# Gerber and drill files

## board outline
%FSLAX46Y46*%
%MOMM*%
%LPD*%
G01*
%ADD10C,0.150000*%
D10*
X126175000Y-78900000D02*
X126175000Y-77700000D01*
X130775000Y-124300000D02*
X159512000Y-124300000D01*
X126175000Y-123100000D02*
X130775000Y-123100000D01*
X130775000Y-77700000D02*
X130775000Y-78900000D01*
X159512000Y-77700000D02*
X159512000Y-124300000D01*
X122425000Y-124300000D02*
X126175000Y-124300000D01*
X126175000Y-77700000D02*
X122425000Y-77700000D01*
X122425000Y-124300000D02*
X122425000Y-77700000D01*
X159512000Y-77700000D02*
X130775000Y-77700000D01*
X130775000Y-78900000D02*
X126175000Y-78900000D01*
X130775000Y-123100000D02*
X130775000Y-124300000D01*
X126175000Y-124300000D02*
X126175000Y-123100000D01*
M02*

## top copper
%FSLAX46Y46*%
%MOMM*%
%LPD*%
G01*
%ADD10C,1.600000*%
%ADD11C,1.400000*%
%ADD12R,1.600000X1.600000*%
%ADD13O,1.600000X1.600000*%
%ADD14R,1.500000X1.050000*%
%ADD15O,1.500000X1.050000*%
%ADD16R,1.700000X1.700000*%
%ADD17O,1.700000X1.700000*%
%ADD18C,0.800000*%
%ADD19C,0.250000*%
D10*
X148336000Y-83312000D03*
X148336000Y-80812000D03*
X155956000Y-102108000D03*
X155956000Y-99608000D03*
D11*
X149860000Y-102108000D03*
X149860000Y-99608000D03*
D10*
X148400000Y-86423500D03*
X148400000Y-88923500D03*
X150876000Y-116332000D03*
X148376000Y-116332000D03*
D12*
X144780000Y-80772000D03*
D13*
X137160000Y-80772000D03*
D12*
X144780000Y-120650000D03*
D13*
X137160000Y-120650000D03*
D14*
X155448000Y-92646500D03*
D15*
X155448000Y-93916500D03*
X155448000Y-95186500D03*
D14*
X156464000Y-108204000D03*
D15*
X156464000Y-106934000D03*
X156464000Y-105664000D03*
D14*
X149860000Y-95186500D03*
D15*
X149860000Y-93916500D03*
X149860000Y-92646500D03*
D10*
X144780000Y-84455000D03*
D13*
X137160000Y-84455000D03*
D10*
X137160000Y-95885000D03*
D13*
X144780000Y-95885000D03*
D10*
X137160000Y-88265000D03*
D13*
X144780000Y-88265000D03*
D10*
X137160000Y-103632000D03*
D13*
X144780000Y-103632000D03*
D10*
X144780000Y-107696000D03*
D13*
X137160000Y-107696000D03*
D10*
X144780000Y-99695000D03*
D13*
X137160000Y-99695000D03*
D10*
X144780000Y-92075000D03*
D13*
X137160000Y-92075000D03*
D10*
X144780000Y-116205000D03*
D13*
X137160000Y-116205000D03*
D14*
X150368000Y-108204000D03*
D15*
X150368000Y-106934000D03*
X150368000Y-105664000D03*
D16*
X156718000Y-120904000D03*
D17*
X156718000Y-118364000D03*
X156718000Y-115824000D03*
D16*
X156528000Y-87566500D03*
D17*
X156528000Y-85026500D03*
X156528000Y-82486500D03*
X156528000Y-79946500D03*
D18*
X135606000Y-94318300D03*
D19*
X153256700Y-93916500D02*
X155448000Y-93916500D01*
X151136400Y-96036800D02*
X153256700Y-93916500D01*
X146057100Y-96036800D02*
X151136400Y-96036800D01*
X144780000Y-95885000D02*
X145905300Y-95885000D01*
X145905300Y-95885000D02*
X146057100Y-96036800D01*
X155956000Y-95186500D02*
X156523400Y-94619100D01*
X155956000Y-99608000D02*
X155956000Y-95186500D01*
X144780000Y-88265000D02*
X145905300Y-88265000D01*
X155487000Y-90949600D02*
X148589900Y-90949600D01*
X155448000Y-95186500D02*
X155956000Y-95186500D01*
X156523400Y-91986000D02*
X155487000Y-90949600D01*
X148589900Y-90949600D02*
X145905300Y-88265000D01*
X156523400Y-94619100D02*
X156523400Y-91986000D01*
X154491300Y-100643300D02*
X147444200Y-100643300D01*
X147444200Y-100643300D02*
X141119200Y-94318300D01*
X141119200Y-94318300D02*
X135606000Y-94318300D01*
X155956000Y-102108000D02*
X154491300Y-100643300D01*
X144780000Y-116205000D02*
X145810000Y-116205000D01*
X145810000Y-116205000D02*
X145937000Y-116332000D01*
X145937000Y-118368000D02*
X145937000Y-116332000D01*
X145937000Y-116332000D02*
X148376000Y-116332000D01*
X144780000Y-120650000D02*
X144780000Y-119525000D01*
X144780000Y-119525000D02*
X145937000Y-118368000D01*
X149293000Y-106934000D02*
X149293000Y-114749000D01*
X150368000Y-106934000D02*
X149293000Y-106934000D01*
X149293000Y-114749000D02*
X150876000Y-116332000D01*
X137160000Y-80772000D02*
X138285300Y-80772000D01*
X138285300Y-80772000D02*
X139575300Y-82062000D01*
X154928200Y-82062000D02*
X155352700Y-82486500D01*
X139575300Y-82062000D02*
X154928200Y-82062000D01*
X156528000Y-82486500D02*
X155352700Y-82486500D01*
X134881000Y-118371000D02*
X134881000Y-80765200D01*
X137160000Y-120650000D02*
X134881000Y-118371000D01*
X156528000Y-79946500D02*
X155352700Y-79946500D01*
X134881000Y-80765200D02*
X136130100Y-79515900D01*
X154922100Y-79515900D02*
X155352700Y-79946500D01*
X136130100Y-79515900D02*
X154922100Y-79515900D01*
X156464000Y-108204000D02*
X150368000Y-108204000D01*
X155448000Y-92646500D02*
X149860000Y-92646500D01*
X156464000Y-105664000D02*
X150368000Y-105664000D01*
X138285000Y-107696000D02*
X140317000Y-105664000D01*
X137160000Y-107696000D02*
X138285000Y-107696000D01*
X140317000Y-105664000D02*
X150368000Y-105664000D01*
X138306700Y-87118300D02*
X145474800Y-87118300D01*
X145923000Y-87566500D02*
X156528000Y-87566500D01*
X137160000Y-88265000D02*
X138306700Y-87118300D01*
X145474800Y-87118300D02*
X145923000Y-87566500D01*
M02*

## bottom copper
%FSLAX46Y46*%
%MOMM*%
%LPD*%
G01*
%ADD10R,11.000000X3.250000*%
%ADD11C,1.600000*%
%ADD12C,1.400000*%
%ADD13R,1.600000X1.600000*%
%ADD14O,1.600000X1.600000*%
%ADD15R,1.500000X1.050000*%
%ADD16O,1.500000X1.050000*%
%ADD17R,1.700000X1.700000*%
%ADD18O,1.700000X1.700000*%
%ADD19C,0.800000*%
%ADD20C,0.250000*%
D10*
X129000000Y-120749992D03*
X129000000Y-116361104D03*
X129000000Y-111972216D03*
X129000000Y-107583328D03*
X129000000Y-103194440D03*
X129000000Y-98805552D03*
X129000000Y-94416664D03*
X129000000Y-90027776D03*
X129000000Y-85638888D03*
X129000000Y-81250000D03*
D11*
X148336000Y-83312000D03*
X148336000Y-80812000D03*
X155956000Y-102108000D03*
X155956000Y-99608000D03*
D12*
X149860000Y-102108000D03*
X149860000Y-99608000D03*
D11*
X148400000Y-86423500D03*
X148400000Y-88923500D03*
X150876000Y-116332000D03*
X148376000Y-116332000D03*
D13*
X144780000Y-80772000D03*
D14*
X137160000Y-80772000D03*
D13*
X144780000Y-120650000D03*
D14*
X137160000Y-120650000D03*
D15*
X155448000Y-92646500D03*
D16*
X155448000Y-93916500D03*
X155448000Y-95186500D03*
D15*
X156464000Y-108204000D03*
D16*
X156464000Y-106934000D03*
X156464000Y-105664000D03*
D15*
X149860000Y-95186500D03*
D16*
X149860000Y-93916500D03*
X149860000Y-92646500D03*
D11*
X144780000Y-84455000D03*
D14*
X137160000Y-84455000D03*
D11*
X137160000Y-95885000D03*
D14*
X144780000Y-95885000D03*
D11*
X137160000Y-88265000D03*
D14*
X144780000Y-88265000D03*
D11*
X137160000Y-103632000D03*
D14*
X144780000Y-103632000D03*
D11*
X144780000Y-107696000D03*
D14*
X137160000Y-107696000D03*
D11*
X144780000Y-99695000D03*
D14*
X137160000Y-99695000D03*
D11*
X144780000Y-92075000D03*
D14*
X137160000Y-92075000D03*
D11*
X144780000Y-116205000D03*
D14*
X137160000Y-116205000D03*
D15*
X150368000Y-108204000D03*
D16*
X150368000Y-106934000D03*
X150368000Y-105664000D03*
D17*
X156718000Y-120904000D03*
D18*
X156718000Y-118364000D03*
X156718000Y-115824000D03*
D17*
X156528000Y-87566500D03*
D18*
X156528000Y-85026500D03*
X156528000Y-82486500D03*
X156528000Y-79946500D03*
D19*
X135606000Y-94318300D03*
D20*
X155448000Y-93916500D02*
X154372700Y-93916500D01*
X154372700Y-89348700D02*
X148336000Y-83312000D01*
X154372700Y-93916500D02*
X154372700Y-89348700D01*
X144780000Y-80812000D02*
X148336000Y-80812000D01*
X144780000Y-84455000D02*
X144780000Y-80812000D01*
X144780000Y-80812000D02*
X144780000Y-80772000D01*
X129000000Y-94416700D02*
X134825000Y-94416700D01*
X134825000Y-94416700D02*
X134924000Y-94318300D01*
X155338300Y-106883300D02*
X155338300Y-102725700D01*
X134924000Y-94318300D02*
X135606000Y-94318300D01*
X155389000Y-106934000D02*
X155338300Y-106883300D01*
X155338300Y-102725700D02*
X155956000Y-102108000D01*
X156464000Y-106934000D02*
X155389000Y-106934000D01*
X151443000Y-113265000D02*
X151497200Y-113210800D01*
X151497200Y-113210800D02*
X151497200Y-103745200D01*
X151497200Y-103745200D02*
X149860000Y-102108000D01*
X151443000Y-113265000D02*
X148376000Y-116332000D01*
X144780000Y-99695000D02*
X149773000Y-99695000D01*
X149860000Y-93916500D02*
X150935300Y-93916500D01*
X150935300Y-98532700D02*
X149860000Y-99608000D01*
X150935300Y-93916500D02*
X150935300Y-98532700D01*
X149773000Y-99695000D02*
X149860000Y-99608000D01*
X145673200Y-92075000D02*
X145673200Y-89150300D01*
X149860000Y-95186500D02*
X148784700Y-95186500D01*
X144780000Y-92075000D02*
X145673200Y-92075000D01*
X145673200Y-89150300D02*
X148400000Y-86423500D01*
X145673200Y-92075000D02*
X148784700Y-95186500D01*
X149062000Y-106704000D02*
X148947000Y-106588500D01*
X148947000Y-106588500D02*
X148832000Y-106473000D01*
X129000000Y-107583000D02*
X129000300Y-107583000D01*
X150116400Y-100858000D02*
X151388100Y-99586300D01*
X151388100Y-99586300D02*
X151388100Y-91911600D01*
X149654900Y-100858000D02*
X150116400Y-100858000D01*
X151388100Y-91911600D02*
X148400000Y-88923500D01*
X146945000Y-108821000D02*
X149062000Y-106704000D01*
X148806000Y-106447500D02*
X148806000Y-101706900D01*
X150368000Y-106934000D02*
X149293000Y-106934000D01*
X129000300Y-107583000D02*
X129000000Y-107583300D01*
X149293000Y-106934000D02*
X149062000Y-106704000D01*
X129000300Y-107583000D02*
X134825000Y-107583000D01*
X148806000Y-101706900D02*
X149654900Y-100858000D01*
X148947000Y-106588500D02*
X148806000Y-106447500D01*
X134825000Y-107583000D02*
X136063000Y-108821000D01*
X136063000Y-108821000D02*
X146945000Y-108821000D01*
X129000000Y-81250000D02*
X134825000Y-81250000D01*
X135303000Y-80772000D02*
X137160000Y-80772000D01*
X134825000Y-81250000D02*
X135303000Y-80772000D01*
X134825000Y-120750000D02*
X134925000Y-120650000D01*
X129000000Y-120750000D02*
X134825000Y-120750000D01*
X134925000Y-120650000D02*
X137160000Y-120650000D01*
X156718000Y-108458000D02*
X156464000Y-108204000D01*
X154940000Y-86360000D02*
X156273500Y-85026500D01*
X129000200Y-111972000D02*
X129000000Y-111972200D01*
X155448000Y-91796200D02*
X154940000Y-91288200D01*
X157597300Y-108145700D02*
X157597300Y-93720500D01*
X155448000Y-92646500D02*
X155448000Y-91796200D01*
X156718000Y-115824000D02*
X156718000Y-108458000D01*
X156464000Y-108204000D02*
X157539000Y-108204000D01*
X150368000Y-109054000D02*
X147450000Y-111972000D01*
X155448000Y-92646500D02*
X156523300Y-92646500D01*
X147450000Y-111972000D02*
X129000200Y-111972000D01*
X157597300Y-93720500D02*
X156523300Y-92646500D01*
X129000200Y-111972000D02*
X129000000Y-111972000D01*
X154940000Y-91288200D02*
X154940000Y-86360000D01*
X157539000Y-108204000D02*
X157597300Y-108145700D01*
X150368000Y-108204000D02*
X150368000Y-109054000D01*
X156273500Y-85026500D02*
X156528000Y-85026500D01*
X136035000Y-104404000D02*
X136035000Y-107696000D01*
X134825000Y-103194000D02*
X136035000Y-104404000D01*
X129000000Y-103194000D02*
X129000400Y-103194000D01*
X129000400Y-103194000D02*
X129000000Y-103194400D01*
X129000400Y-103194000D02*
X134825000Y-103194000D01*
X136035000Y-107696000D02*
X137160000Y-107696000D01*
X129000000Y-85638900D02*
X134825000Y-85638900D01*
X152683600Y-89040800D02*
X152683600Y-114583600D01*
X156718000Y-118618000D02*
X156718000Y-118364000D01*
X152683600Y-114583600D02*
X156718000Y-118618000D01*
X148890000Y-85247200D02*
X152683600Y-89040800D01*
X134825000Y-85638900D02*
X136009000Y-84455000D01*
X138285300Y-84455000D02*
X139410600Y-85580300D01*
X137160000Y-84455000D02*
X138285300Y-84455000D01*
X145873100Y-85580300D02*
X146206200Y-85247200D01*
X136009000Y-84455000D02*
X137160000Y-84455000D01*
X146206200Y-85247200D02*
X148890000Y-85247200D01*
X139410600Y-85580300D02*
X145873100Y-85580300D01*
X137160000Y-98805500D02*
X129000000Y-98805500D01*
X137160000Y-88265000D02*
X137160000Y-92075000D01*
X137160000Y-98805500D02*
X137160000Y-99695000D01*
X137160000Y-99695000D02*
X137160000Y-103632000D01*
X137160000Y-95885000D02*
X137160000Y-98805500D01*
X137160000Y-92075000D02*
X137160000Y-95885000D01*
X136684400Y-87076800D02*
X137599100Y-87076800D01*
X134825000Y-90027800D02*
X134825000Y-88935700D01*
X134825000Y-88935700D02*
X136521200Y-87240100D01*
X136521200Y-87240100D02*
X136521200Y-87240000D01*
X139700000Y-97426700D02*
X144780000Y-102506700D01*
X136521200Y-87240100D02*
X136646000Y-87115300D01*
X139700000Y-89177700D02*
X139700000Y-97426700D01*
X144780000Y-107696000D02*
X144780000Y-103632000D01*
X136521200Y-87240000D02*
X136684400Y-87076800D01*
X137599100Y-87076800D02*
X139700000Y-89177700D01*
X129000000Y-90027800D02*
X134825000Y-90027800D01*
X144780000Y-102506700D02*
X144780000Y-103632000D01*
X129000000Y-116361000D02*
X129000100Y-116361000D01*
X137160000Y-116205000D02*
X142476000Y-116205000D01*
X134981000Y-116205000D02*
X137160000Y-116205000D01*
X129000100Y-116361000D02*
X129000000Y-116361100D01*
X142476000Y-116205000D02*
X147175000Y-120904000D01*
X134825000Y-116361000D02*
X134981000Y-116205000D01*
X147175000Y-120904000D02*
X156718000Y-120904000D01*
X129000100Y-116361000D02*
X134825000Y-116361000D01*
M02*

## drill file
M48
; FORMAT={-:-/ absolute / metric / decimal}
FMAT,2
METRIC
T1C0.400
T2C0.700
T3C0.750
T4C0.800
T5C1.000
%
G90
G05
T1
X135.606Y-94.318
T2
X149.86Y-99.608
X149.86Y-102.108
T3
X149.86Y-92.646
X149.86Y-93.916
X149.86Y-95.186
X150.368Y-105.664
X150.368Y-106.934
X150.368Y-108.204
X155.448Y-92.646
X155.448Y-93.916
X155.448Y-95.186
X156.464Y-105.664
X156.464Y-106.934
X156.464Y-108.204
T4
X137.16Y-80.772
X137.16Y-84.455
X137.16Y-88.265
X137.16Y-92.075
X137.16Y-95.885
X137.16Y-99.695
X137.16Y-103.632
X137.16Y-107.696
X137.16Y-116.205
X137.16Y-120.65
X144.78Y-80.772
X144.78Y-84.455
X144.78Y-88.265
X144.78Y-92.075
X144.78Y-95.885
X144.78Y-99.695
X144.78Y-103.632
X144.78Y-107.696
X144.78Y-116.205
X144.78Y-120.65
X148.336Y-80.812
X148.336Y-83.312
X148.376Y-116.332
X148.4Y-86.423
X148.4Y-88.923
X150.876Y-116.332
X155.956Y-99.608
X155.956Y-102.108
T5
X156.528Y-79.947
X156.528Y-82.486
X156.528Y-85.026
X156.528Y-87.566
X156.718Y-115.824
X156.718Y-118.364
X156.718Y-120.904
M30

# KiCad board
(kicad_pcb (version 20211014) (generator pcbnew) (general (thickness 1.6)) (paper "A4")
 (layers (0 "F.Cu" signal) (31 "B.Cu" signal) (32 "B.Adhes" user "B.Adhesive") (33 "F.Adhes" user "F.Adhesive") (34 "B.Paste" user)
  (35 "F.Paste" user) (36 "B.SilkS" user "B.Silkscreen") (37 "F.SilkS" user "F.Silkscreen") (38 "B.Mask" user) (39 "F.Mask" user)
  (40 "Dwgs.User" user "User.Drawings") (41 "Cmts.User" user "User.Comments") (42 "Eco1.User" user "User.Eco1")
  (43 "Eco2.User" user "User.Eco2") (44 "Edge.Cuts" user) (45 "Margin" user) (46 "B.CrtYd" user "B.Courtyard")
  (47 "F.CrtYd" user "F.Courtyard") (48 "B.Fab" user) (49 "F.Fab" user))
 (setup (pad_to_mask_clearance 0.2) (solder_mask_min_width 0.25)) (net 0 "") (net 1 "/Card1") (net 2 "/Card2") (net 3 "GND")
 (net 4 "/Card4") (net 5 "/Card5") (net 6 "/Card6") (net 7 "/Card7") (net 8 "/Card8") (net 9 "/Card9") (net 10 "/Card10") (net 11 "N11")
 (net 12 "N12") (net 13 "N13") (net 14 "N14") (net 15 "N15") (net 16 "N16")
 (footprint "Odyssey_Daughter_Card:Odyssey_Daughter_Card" (layer "F.Cu") (at 129 101)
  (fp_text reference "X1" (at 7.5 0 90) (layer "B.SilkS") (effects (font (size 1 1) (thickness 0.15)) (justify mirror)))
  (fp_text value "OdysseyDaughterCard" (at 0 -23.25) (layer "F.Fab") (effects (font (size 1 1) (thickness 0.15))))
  (pad "1" smd rect locked (at 0 19.749992) (size 11 3.25) (layers "B.Cu" "B.Mask") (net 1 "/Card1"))
  (pad "2" smd rect locked (at 0 15.361104) (size 11 3.25) (layers "B.Cu" "B.Mask") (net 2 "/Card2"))
  (pad "3" smd rect locked (at 0 10.972216) (size 11 3.25) (layers "B.Cu" "B.Mask") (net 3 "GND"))
  (pad "4" smd rect locked (at 0 6.583328) (size 11 3.25) (layers "B.Cu" "B.Mask") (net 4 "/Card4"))
  (pad "5" smd rect locked (at 0 2.19444) (size 11 3.25) (layers "B.Cu" "B.Mask") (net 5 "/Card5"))
  (pad "6" smd rect locked (at 0 -2.194448) (size 11 3.25) (layers "B.Cu" "B.Mask") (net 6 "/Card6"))
  (pad "7" smd rect locked (at 0 -6.583336) (size 11 3.25) (layers "B.Cu" "B.Mask") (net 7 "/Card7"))
  (pad "8" smd rect locked (at 0 -10.972224) (size 11 3.25) (layers "B.Cu" "B.Mask") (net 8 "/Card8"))
  (pad "9" smd rect locked (at 0 -15.361112) (size 11 3.25) (layers "B.Cu" "B.Mask") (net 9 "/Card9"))
  (pad "10" smd rect locked (at 0 -19.75) (size 11 3.25) (layers "B.Cu" "B.Mask") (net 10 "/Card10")))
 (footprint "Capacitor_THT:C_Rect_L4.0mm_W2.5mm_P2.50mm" (layer "F.Cu") (at 148.336 83.312 90)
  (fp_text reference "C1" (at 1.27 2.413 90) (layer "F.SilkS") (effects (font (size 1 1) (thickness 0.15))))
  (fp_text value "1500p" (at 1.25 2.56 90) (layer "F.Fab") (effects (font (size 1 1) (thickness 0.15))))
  (pad "1" thru_hole circle locked (at 0 0 90) (size 1.6 1.6) (drill 0.8) (layers *.Cu *.Mask) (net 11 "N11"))
  (pad "2" thru_hole circle locked (at 2.5 0 90) (size 1.6 1.6) (drill 0.8) (layers *.Cu *.Mask) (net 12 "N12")))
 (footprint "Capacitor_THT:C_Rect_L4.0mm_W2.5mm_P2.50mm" (layer "F.Cu") (at 155.956 102.108 90)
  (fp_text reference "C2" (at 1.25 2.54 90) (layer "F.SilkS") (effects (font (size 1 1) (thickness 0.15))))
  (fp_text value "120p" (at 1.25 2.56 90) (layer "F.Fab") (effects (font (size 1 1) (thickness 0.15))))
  (pad "1" thru_hole circle locked (at 0 0 90) (size 1.6 1.6) (drill 0.8) (layers *.Cu *.Mask) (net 7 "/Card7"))
  (pad "2" thru_hole circle locked (at 2.5 0 90) (size 1.6 1.6) (drill 0.8) (layers *.Cu *.Mask) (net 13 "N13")))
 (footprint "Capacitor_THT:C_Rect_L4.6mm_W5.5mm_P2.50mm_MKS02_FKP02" (layer "F.Cu") (at 149.86 102.108 90)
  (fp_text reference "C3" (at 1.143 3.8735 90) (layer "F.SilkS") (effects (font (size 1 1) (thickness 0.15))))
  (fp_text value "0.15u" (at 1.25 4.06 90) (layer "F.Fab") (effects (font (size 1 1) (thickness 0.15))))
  (pad "1" thru_hole circle locked (at 0 0 90) (size 1.4 1.4) (drill 0.7) (layers *.Cu *.Mask) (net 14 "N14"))
  (pad "2" thru_hole circle locked (at 2.5 0 90) (size 1.4 1.4) (drill 0.7) (layers *.Cu *.Mask) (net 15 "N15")))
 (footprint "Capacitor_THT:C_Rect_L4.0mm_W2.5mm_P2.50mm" (layer "F.Cu") (at 148.4 86.4235 -90)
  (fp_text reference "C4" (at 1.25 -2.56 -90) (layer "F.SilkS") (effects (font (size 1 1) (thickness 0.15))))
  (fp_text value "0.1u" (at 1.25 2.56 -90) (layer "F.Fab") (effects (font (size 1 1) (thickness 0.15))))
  (pad "1" thru_hole circle locked (at 0 0 270) (size 1.6 1.6) (drill 0.8) (layers *.Cu *.Mask) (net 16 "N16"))
  (pad "2" thru_hole circle locked (at 2.5 0 270) (size 1.6 1.6) (drill 0.8) (layers *.Cu *.Mask) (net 4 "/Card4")))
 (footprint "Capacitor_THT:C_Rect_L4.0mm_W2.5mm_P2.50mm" (layer "F.Cu") (at 150.876 116.332 180)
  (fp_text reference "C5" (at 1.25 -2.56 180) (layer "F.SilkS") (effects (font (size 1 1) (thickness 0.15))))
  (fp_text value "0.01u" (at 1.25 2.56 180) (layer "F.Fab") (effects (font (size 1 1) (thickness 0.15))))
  (pad "1" thru_hole circle locked (at 0 0 180) (size 1.6 1.6) (drill 0.8) (layers *.Cu *.Mask) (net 4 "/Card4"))
  (pad "2" thru_hole circle locked (at 2.5 0 180) (size 1.6 1.6) (drill 0.8) (layers *.Cu *.Mask) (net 14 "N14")))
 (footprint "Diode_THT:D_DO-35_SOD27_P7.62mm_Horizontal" (layer "F.Cu") (at 144.78 80.772 180)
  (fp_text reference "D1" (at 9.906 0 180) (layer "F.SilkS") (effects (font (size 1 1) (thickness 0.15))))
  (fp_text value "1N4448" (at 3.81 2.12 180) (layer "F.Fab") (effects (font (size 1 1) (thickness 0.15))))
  (pad "1" thru_hole rect locked (at 0 0 180) (size 1.6 1.6) (drill 0.8) (layers *.Cu *.Mask) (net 12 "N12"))
  (pad "2" thru_hole oval locked (at 7.62 0 180) (size 1.6 1.6) (drill 0.8) (layers *.Cu *.Mask) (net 10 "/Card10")))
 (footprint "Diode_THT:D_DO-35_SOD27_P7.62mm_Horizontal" (layer "F.Cu") (at 144.78 120.65 180)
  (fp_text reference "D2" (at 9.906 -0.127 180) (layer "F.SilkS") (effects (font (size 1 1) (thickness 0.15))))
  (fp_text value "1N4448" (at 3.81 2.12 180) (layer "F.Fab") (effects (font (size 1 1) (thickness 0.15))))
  (pad "1" thru_hole rect locked (at 0 0 180) (size 1.6 1.6) (drill 0.8) (layers *.Cu *.Mask) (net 14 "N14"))
  (pad "2" thru_hole oval locked (at 7.62 0 180) (size 1.6 1.6) (drill 0.8) (layers *.Cu *.Mask) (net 1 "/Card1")))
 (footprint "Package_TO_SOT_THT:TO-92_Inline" (layer "F.Cu") (at 155.448 92.6465 -90)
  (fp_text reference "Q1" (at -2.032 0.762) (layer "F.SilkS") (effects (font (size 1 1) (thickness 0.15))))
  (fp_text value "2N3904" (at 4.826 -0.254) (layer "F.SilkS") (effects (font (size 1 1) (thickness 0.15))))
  (pad "1" thru_hole rect locked (at 0 0 270) (size 1.05 1.5) (drill 0.75) (layers *.Cu *.Mask) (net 3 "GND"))
  (pad "2" thru_hole oval locked (at 1.27 0 270) (size 1.05 1.5) (drill 0.75) (layers *.Cu *.Mask) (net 11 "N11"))
  (pad "3" thru_hole oval locked (at 2.54 0 270) (size 1.05 1.5) (drill 0.75) (layers *.Cu *.Mask) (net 13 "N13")))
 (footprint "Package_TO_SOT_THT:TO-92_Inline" (layer "F.Cu") (at 156.464 108.204 90)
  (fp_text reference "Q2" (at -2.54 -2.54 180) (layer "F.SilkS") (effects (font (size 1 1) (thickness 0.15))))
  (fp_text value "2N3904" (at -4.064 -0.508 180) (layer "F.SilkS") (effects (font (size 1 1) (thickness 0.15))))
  (pad "1" thru_hole rect locked (at 0 0 90) (size 1.05 1.5) (drill 0.75) (layers *.Cu *.Mask) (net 3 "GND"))
  (pad "2" thru_hole oval locked (at 1.27 0 90) (size 1.05 1.5) (drill 0.75) (layers *.Cu *.Mask) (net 7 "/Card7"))
  (pad "3" thru_hole oval locked (at 2.54 0 90) (size 1.05 1.5) (drill 0.75) (layers *.Cu *.Mask) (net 5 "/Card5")))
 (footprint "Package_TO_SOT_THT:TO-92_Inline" (layer "F.Cu") (at 149.86 95.1865 90)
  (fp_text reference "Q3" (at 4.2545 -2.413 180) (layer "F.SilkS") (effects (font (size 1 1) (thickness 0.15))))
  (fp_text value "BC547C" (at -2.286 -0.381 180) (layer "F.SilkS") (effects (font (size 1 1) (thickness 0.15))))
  (pad "1" thru_hole rect locked (at 0 0 90) (size 1.05 1.5) (drill 0.75) (layers *.Cu *.Mask) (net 16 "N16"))
  (pad "2" thru_hole oval locked (at 1.27 0 90) (size 1.05 1.5) (drill 0.75) (layers *.Cu *.Mask) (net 15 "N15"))
  (pad "3" thru_hole oval locked (at 2.54 0 90) (size 1.05 1.5) (drill 0.75) (layers *.Cu *.Mask) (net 3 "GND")))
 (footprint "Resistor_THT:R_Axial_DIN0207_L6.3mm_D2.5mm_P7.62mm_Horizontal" (layer "F.Cu") (at 144.78 84.455 180)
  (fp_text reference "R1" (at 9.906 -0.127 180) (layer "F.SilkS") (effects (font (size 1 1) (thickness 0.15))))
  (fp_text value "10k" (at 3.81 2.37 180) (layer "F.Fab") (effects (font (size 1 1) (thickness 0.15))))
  (pad "1" thru_hole circle locked (at 0 0 180) (size 1.6 1.6) (drill 0.8) (layers *.Cu *.Mask) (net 12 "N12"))
  (pad "2" thru_hole oval locked (at 7.62 0 180) (size 1.6 1.6) (drill 0.8) (layers *.Cu *.Mask) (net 9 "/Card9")))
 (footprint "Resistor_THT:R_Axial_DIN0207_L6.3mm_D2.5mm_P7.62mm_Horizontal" (layer "F.Cu") (at 137.16 95.885)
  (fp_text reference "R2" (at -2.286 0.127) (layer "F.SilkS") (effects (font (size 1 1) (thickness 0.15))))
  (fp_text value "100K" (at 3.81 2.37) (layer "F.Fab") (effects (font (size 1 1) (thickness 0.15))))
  (pad "1" thru_hole circle locked (at 0 0) (size 1.6 1.6) (drill 0.8) (layers *.Cu *.Mask) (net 6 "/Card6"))
  (pad "2" thru_hole oval locked (at 7.62 0) (size 1.6 1.6) (drill 0.8) (layers *.Cu *.Mask) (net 11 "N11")))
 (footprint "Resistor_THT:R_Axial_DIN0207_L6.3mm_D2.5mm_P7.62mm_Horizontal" (layer "F.Cu") (at 137.16 88.265)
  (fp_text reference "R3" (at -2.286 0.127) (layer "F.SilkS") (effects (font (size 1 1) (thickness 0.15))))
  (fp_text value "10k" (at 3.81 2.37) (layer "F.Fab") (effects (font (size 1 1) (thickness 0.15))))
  (pad "1" thru_hole circle locked (at 0 0) (size 1.6 1.6) (drill 0.8) (layers *.Cu *.Mask) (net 6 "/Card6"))
  (pad "2" thru_hole oval locked (at 7.62 0) (size 1.6 1.6) (drill 0.8) (layers *.Cu *.Mask) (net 13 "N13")))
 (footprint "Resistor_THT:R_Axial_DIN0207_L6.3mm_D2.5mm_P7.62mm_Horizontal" (layer "F.Cu") (at 137.16 103.632)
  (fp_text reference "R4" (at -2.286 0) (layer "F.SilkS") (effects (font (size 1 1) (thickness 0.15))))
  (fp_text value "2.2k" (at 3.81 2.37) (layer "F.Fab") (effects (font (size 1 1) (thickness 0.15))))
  (pad "1" thru_hole circle locked (at 0 0) (size 1.6 1.6) (drill 0.8) (layers *.Cu *.Mask) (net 6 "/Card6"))
  (pad "2" thru_hole oval locked (at 7.62 0) (size 1.6 1.6) (drill 0.8) (layers *.Cu *.Mask) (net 8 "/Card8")))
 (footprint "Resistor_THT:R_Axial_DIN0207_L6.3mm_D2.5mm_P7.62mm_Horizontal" (layer "F.Cu") (at 144.78 107.696 180)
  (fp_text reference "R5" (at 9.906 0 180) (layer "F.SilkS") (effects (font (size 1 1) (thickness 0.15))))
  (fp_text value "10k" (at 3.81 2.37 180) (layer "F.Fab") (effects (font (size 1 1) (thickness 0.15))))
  (pad "1" thru_hole circle locked (at 0 0 180) (size 1.6 1.6) (drill 0.8) (layers *.Cu *.Mask) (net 8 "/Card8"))
  (pad "2" thru_hole oval locked (at 7.62 0 180) (size 1.6 1.6) (drill 0.8) (layers *.Cu *.Mask) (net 5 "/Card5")))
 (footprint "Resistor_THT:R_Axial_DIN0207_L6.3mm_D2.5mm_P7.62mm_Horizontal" (layer "F.Cu") (at 144.78 99.695 180)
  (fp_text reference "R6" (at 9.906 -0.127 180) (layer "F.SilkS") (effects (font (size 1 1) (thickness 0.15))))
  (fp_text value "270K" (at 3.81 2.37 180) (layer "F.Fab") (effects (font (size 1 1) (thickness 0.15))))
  (pad "1" thru_hole circle locked (at 0 0 180) (size 1.6 1.6) (drill 0.8) (layers *.Cu *.Mask) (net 15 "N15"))
  (pad "2" thru_hole oval locked (at 7.62 0 180) (size 1.6 1.6) (drill 0.8) (layers *.Cu *.Mask) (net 6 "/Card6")))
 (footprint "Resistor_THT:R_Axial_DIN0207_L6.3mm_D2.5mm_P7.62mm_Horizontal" (layer "F.Cu") (at 144.78 92.075 180)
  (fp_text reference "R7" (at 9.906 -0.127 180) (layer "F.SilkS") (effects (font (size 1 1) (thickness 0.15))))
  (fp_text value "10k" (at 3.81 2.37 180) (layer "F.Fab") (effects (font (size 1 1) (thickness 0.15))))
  (pad "1" thru_hole circle locked (at 0 0 180) (size 1.6 1.6) (drill 0.8) (layers *.Cu *.Mask) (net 16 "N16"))
  (pad "2" thru_hole oval locked (at 7.62 0 180) (size 1.6 1.6) (drill 0.8) (layers *.Cu *.Mask) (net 6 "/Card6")))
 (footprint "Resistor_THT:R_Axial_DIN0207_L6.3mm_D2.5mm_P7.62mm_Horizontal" (layer "F.Cu") (at 144.78 116.205 180)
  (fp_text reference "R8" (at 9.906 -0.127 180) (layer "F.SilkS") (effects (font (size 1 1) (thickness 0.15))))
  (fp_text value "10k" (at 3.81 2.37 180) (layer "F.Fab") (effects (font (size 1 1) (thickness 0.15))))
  (pad "1" thru_hole circle locked (at 0 0 180) (size 1.6 1.6) (drill 0.8) (layers *.Cu *.Mask) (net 14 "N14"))
  (pad "2" thru_hole oval locked (at 7.62 0 180) (size 1.6 1.6) (drill 0.8) (layers *.Cu *.Mask) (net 2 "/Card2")))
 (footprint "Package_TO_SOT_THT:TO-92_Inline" (layer "F.Cu") (at 150.368 108.204 90)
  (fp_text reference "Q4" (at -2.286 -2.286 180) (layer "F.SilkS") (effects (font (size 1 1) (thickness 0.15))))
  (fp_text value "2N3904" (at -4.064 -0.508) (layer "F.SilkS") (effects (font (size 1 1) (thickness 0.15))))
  (pad "1" thru_hole rect locked (at 0 0 90) (size 1.05 1.5) (drill 0.75) (layers *.Cu *.Mask) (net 3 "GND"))
  (pad "2" thru_hole oval locked (at 1.27 0 90) (size 1.05 1.5) (drill 0.75) (layers *.Cu *.Mask) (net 4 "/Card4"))
  (pad "3" thru_hole oval locked (at 2.54 0 90) (size 1.05 1.5) (drill 0.75) (layers *.Cu *.Mask) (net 5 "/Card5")))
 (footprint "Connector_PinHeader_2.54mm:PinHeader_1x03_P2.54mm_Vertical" (layer "F.Cu") (at 156.718 120.904 180)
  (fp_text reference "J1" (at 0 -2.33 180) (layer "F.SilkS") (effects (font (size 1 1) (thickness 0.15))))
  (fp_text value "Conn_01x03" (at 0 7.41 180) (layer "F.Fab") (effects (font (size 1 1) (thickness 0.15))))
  (pad "1" thru_hole rect locked (at 0 0 180) (size 1.7 1.7) (drill 1) (layers *.Cu *.Mask) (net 2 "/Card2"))
  (pad "2" thru_hole oval locked (at 0 2.54 180) (size 1.7 1.7) (drill 1) (layers *.Cu *.Mask) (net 9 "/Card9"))
  (pad "3" thru_hole oval locked (at 0 5.08 180) (size 1.7 1.7) (drill 1) (layers *.Cu *.Mask) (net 3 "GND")))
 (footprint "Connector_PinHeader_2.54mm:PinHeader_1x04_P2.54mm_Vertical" (layer "F.Cu") (at 156.528 87.5665 180)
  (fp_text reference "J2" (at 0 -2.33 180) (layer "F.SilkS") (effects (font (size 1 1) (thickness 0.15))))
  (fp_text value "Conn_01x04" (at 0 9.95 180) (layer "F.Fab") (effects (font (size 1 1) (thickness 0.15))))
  (pad "1" thru_hole rect locked (at 0 0 180) (size 1.7 1.7) (drill 1) (layers *.Cu *.Mask) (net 6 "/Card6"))
  (pad "2" thru_hole oval locked (at 0 2.54 180) (size 1.7 1.7) (drill 1) (layers *.Cu *.Mask) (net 3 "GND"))
  (pad "3" thru_hole oval locked (at 0 5.08 180) (size 1.7 1.7) (drill 1) (layers *.Cu *.Mask) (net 10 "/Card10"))
  (pad "4" thru_hole oval locked (at 0 7.62 180) (size 1.7 1.7) (drill 1) (layers *.Cu *.Mask) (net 1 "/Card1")))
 (gr_line (start 126.175 78.9) (end 126.175 77.7) (layer "Edge.Cuts") (width 0.15))
 (gr_line (start 130.775 124.3) (end 159.512 124.3) (layer "Edge.Cuts") (width 0.15))
 (gr_line (start 126.175 123.1) (end 130.775 123.1) (layer "Edge.Cuts") (width 0.15))
 (gr_line (start 130.775 77.7) (end 130.775 78.9) (layer "Edge.Cuts") (width 0.15))
 (gr_line (start 159.512 77.7) (end 159.512 124.3) (layer "Edge.Cuts") (width 0.15))
 (gr_line (start 122.425 124.3) (end 126.175 124.3) (layer "Edge.Cuts") (width 0.15))
 (gr_line (start 126.175 77.7) (end 122.425 77.7) (layer "Edge.Cuts") (width 0.15))
 (gr_line (start 122.425 124.3) (end 122.425 77.7) (layer "Edge.Cuts") (width 0.15))
 (gr_line (start 159.512 77.7) (end 130.775 77.7) (layer "Edge.Cuts") (width 0.15))
 (gr_line (start 130.775 78.9) (end 126.175 78.9) (layer "Edge.Cuts") (width 0.15))
 (gr_line (start 130.775 123.1) (end 130.775 124.3) (layer "Edge.Cuts") (width 0.15))
 (gr_line (start 126.175 124.3) (end 126.175 123.1) (layer "Edge.Cuts") (width 0.15))
 (segment (start 153.2567 93.9165) (end 155.448 93.9165) (width 0.25) (layer "F.Cu") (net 11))
 (segment (start 151.1364 96.0368) (end 153.2567 93.9165) (width 0.25) (layer "F.Cu") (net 11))
 (segment (start 146.0571 96.0368) (end 151.1364 96.0368) (width 0.25) (layer "F.Cu") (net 11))
 (segment (start 144.78 95.885) (end 145.9053 95.885) (width 0.25) (layer "F.Cu") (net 11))
 (segment (start 145.9053 95.885) (end 146.0571 96.0368) (width 0.25) (layer "F.Cu") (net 11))
 (segment (start 155.448 93.9165) (end 154.3727 93.9165) (width 0.25) (layer "B.Cu") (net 11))
 (segment (start 154.3727 89.3487) (end 148.336 83.312) (width 0.25) (layer "B.Cu") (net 11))
 (segment (start 154.3727 93.9165) (end 154.3727 89.3487) (width 0.25) (layer "B.Cu") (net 11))
 (segment (start 144.78 80.812) (end 148.336 80.812) (width 0.25) (layer "B.Cu") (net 12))
 (segment (start 144.78 84.455) (end 144.78 80.812) (width 0.25) (layer "B.Cu") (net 12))
 (segment (start 144.78 80.812) (end 144.78 80.772) (width 0.25) (layer "B.Cu") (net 12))
 (segment (start 155.956 95.1865) (end 156.5234 94.6191) (width 0.25) (layer "F.Cu") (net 13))
 (segment (start 155.956 99.608) (end 155.956 95.1865) (width 0.25) (layer "F.Cu") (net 13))
 (segment (start 144.78 88.265) (end 145.9053 88.265) (width 0.25) (layer "F.Cu") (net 13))
 (segment (start 155.487 90.9496) (end 148.5899 90.9496) (width 0.25) (layer "F.Cu") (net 13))
 (segment (start 155.448 95.1865) (end 155.956 95.1865) (width 0.25) (layer "F.Cu") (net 13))
 (segment (start 156.5234 91.986) (end 155.487 90.9496) (width 0.25) (layer "F.Cu") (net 13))
 (segment (start 148.5899 90.9496) (end 145.9053 88.265) (width 0.25) (layer "F.Cu") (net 13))
 (segment (start 156.5234 94.6191) (end 156.5234 91.986) (width 0.25) (layer "F.Cu") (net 13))
 (segment (start 154.4913 100.6433) (end 147.4442 100.6433) (width 0.25) (layer "F.Cu") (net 7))
 (segment (start 147.4442 100.6433) (end 141.1192 94.3183) (width 0.25) (layer "F.Cu") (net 7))
 (segment (start 141.1192 94.3183) (end 135.606 94.3183) (width 0.25) (layer "F.Cu") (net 7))
 (segment (start 155.956 102.108) (end 154.4913 100.6433) (width 0.25) (layer "F.Cu") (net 7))
 (via (at 135.606 94.3183) (size 0.8) (drill 0.4) (layers "F.Cu" "B.Cu") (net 7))
 (segment (start 129 94.4167) (end 134.825 94.4167) (width 0.25) (layer "B.Cu") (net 7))
 (segment (start 134.825 94.4167) (end 134.924 94.3183) (width 0.25) (layer "B.Cu") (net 7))
 (segment (start 155.3383 106.8833) (end 155.3383 102.7257) (width 0.25) (layer "B.Cu") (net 7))
 (segment (start 134.924 94.3183) (end 135.606 94.3183) (width 0.25) (layer "B.Cu") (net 7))
 (segment (start 155.389 106.934) (end 155.3383 106.8833) (width 0.25) (layer "B.Cu") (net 7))
 (segment (start 155.3383 102.7257) (end 155.956 102.108) (width 0.25) (layer "B.Cu") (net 7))
 (segment (start 156.464 106.934) (end 155.389 106.934) (width 0.25) (layer "B.Cu") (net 7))
 (segment (start 144.78 116.205) (end 145.81 116.205) (width 0.25) (layer "F.Cu") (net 14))
 (segment (start 145.81 116.205) (end 145.937 116.332) (width 0.25) (layer "F.Cu") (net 14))
 (segment (start 145.937 118.368) (end 145.937 116.332) (width 0.25) (layer "F.Cu") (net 14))
 (segment (start 145.937 116.332) (end 148.376 116.332) (width 0.25) (layer "F.Cu") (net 14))
 (segment (start 144.78 120.65) (end 144.78 119.525) (width 0.25) (layer "F.Cu") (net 14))
 (segment (start 144.78 119.525) (end 145.937 118.368) (width 0.25) (layer "F.Cu") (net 14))
 (segment (start 151.443 113.265) (end 151.4972 113.2108) (width 0.25) (layer "B.Cu") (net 14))
 (segment (start 151.4972 113.2108) (end 151.4972 103.7452) (width 0.25) (layer "B.Cu") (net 14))
 (segment (start 151.4972 103.7452) (end 149.86 102.108) (width 0.25) (layer "B.Cu") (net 14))
 (segment (start 151.443 113.265) (end 148.376 116.332) (width 0.25) (layer "B.Cu") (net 14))
 (segment (start 144.78 99.695) (end 149.773 99.695) (width 0.25) (layer "B.Cu") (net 15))
 (segment (start 149.86 93.9165) (end 150.9353 93.9165) (width 0.25) (layer "B.Cu") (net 15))
 (segment (start 150.9353 98.5327) (end 149.86 99.608) (width 0.25) (layer "B.Cu") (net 15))
 (segment (start 150.9353 93.9165) (end 150.9353 98.5327) (width 0.25) (layer "B.Cu") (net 15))
 (segment (start 149.773 99.695) (end 149.86 99.608) (width 0.25) (layer "B.Cu") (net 15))
 (segment (start 145.6732 92.075) (end 145.6732 89.1503) (width 0.25) (layer "B.Cu") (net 16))
 (segment (start 149.86 95.1865) (end 148.7847 95.1865) (width 0.25) (layer "B.Cu") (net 16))
 (segment (start 144.78 92.075) (end 145.6732 92.075) (width 0.25) (layer "B.Cu") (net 16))
 (segment (start 145.6732 89.1503) (end 148.4 86.4235) (width 0.25) (layer "B.Cu") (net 16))
 (segment (start 145.6732 92.075) (end 148.7847 95.1865) (width 0.25) (layer "B.Cu") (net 16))
 (segment (start 149.293 106.934) (end 149.293 114.749) (width 0.25) (layer "F.Cu") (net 4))
 (segment (start 150.368 106.934) (end 149.293 106.934) (width 0.25) (layer "F.Cu") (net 4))
 (segment (start 149.293 114.749) (end 150.876 116.332) (width 0.25) (layer "F.Cu") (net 4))
 (segment (start 149.062 106.704) (end 148.947 106.5885) (width 0.25) (layer "B.Cu") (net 4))
 (segment (start 148.947 106.5885) (end 148.832 106.473) (width 0.25) (layer "B.Cu") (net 4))
 (segment (start 129 107.583) (end 129.0003 107.583) (width 0.25) (layer "B.Cu") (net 4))
 (segment (start 150.1164 100.858) (end 151.3881 99.5863) (width 0.25) (layer "B.Cu") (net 4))
 (segment (start 151.3881 99.5863) (end 151.3881 91.9116) (width 0.25) (layer "B.Cu") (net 4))
 (segment (start 149.6549 100.858) (end 150.1164 100.858) (width 0.25) (layer "B.Cu") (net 4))
 (segment (start 151.3881 91.9116) (end 148.4 88.9235) (width 0.25) (layer "B.Cu") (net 4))
 (segment (start 146.945 108.821) (end 149.062 106.704) (width 0.25) (layer "B.Cu") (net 4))
 (segment (start 148.806 106.4475) (end 148.806 101.7069) (width 0.25) (layer "B.Cu") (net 4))
 (segment (start 150.368 106.934) (end 149.293 106.934) (width 0.25) (layer "B.Cu") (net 4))
 (segment (start 129.0003 107.583) (end 129 107.5833) (width 0.25) (layer "B.Cu") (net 4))
 (segment (start 149.293 106.934) (end 149.062 106.704) (width 0.25) (layer "B.Cu") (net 4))
 (segment (start 129.0003 107.583) (end 134.825 107.583) (width 0.25) (layer "B.Cu") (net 4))
 (segment (start 148.806 101.7069) (end 149.6549 100.858) (width 0.25) (layer "B.Cu") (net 4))
 (segment (start 148.947 106.5885) (end 148.806 106.4475) (width 0.25) (layer "B.Cu") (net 4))
 (segment (start 134.825 107.583) (end 136.063 108.821) (width 0.25) (layer "B.Cu") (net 4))
 (segment (start 136.063 108.821) (end 146.945 108.821) (width 0.25) (layer "B.Cu") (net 4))
 (segment (start 137.16 80.772) (end 138.2853 80.772) (width 0.25) (layer "F.Cu") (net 10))
 (segment (start 138.2853 80.772) (end 139.5753 82.062) (width 0.25) (layer "F.Cu") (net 10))
 (segment (start 154.9282 82.062) (end 155.3527 82.4865) (width 0.25) (layer "F.Cu") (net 10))
 (segment (start 139.5753 82.062) (end 154.9282 82.062) (width 0.25) (layer "F.Cu") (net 10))
 (segment (start 156.528 82.4865) (end 155.3527 82.4865) (width 0.25) (layer "F.Cu") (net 10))
 (segment (start 129 81.25) (end 134.825 81.25) (width 0.25) (layer "B.Cu") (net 10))
 (segment (start 135.303 80.772) (end 137.16 80.772) (width 0.25) (layer "B.Cu") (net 10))
 (segment (start 134.825 81.25) (end 135.303 80.772) (width 0.25) (layer "B.Cu") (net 10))
 (segment (start 134.881 118.371) (end 134.881 80.7652) (width 0.25) (layer "F.Cu") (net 1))
 (segment (start 137.16 120.65) (end 134.881 118.371) (width 0.25) (layer "F.Cu") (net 1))
 (segment (start 156.528 79.9465) (end 155.3527 79.9465) (width 0.25) (layer "F.Cu") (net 1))
 (segment (start 134.881 80.7652) (end 136.1301 79.5159) (width 0.25) (layer "F.Cu") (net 1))
 (segment (start 154.9221 79.5159) (end 155.3527 79.9465) (width 0.25) (layer "F.Cu") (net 1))
 (segment (start 136.1301 79.5159) (end 154.9221 79.5159) (width 0.25) (layer "F.Cu") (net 1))
 (segment (start 134.825 120.75) (end 134.925 120.65) (width 0.25) (layer "B.Cu") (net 1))
 (segment (start 129 120.75) (end 134.825 120.75) (width 0.25) (layer "B.Cu") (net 1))
 (segment (start 134.925 120.65) (end 137.16 120.65) (width 0.25) (layer "B.Cu") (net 1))
 (segment (start 156.464 108.204) (end 150.368 108.204) (width 0.25) (layer "F.Cu") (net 3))
 (segment (start 155.448 92.6465) (end 149.86 92.6465) (width 0.25) (layer "F.Cu") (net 3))
 (segment (start 156.718 108.458) (end 156.464 108.204) (width 0.25) (layer "B.Cu") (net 3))
 (segment (start 154.94 86.36) (end 156.2735 85.0265) (width 0.25) (layer "B.Cu") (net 3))
 (segment (start 129.0002 111.972) (end 129 111.9722) (width 0.25) (layer "B.Cu") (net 3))
 (segment (start 155.448 91.7962) (end 154.94 91.2882) (width 0.25) (layer "B.Cu") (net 3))
 (segment (start 157.5973 108.1457) (end 157.5973 93.7205) (width 0.25) (layer "B.Cu") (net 3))
 (segment (start 155.448 92.6465) (end 155.448 91.7962) (width 0.25) (layer "B.Cu") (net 3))
 (segment (start 156.718 115.824) (end 156.718 108.458) (width 0.25) (layer "B.Cu") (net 3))
 (segment (start 156.464 108.204) (end 157.539 108.204) (width 0.25) (layer "B.Cu") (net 3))
 (segment (start 150.368 109.054) (end 147.45 111.972) (width 0.25) (layer "B.Cu") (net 3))
 (segment (start 155.448 92.6465) (end 156.5233 92.6465) (width 0.25) (layer "B.Cu") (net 3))
 (segment (start 147.45 111.972) (end 129.0002 111.972) (width 0.25) (layer "B.Cu") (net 3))
 (segment (start 157.5973 93.7205) (end 156.5233 92.6465) (width 0.25) (layer "B.Cu") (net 3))
 (segment (start 129.0002 111.972) (end 129 111.972) (width 0.25) (layer "B.Cu") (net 3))
 (segment (start 154.94 91.2882) (end 154.94 86.36) (width 0.25) (layer "B.Cu") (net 3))
 (segment (start 157.539 108.204) (end 157.5973 108.1457) (width 0.25) (layer "B.Cu") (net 3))
 (segment (start 150.368 108.204) (end 150.368 109.054) (width 0.25) (layer "B.Cu") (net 3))
 (segment (start 156.2735 85.0265) (end 156.528 85.0265) (width 0.25) (layer "B.Cu") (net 3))
 (segment (start 156.464 105.664) (end 150.368 105.664) (width 0.25) (layer "F.Cu") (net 5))
 (segment (start 138.285 107.696) (end 140.317 105.664) (width 0.25) (layer "F.Cu") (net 5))
 (segment (start 137.16 107.696) (end 138.285 107.696) (width 0.25) (layer "F.Cu") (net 5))
 (segment (start 140.317 105.664) (end 150.368 105.664) (width 0.25) (layer "F.Cu") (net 5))
 (segment (start 136.035 104.404) (end 136.035 107.696) (width 0.25) (layer "B.Cu") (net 5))
 (segment (start 134.825 103.194) (end 136.035 104.404) (width 0.25) (layer "B.Cu") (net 5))
 (segment (start 129 103.194) (end 129.0004 103.194) (width 0.25) (layer "B.Cu") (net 5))
 (segment (start 129.0004 103.194) (end 129 103.1944) (width 0.25) (layer "B.Cu") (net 5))
 (segment (start 129.0004 103.194) (end 134.825 103.194) (width 0.25) (layer "B.Cu") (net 5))
 (segment (start 136.035 107.696) (end 137.16 107.696) (width 0.25) (layer "B.Cu") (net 5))
 (segment (start 129 85.6389) (end 134.825 85.6389) (width 0.25) (layer "B.Cu") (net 9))
 (segment (start 152.6836 89.0408) (end 152.6836 114.5836) (width 0.25) (layer "B.Cu") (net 9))
 (segment (start 156.718 118.618) (end 156.718 118.364) (width 0.25) (layer "B.Cu") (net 9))
 (segment (start 152.6836 114.5836) (end 156.718 118.618) (width 0.25) (layer "B.Cu") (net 9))
 (segment (start 148.89 85.2472) (end 152.6836 89.0408) (width 0.25) (layer "B.Cu") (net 9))
 (segment (start 134.825 85.6389) (end 136.009 84.455) (width 0.25) (layer "B.Cu") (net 9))
 (segment (start 138.2853 84.455) (end 139.4106 85.5803) (width 0.25) (layer "B.Cu") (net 9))
 (segment (start 137.16 84.455) (end 138.2853 84.455) (width 0.25) (layer "B.Cu") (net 9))
 (segment (start 145.8731 85.5803) (end 146.2062 85.2472) (width 0.25) (layer "B.Cu") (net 9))
 (segment (start 136.009 84.455) (end 137.16 84.455) (width 0.25) (layer "B.Cu") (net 9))
 (segment (start 146.2062 85.2472) (end 148.89 85.2472) (width 0.25) (layer "B.Cu") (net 9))
 (segment (start 139.4106 85.5803) (end 145.8731 85.5803) (width 0.25) (layer "B.Cu") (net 9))
 (segment (start 138.3067 87.1183) (end 145.4748 87.1183) (width 0.25) (layer "F.Cu") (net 6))
 (segment (start 145.923 87.5665) (end 156.528 87.5665) (width 0.25) (layer "F.Cu") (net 6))
 (segment (start 137.16 88.265) (end 138.3067 87.1183) (width 0.25) (layer "F.Cu") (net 6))
 (segment (start 145.4748 87.1183) (end 145.923 87.5665) (width 0.25) (layer "F.Cu") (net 6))
 (segment (start 137.16 98.8055) (end 129 98.8055) (width 0.25) (layer "B.Cu") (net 6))
 (segment (start 137.16 88.265) (end 137.16 92.075) (width 0.25) (layer "B.Cu") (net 6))
 (segment (start 137.16 98.8055) (end 137.16 99.695) (width 0.25) (layer "B.Cu") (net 6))
 (segment (start 137.16 99.695) (end 137.16 103.632) (width 0.25) (layer "B.Cu") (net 6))
 (segment (start 137.16 95.885) (end 137.16 98.8055) (width 0.25) (layer "B.Cu") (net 6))
 (segment (start 137.16 92.075) (end 137.16 95.885) (width 0.25) (layer "B.Cu") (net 6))
 (segment (start 136.6844 87.0768) (end 137.5991 87.0768) (width 0.25) (layer "B.Cu") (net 8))
 (segment (start 134.825 90.0278) (end 134.825 88.9357) (width 0.25) (layer "B.Cu") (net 8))
 (segment (start 134.825 88.9357) (end 136.5212 87.2401) (width 0.25) (layer "B.Cu") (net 8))
 (segment (start 136.5212 87.2401) (end 136.5212 87.24) (width 0.25) (layer "B.Cu") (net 8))
 (segment (start 139.7 97.4267) (end 144.78 102.5067) (width 0.25) (layer "B.Cu") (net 8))
 (segment (start 136.5212 87.2401) (end 136.646 87.1153) (width 0.25) (layer "B.Cu") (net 8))
 (segment (start 139.7 89.1777) (end 139.7 97.4267) (width 0.25) (layer "B.Cu") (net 8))
 (segment (start 144.78 107.696) (end 144.78 103.632) (width 0.25) (layer "B.Cu") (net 8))
 (segment (start 136.5212 87.24) (end 136.6844 87.0768) (width 0.25) (layer "B.Cu") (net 8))
 (segment (start 137.5991 87.0768) (end 139.7 89.1777) (width 0.25) (layer "B.Cu") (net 8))
 (segment (start 129 90.0278) (end 134.825 90.0278) (width 0.25) (layer "B.Cu") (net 8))
 (segment (start 144.78 102.5067) (end 144.78 103.632) (width 0.25) (layer "B.Cu") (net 8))
 (segment (start 129 116.361) (end 129.0001 116.361) (width 0.25) (layer "B.Cu") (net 2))
 (segment (start 137.16 116.205) (end 142.476 116.205) (width 0.25) (layer "B.Cu") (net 2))
 (segment (start 134.981 116.205) (end 137.16 116.205) (width 0.25) (layer "B.Cu") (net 2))
 (segment (start 129.0001 116.361) (end 129 116.3611) (width 0.25) (layer "B.Cu") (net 2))
 (segment (start 142.476 116.205) (end 147.175 120.904) (width 0.25) (layer "B.Cu") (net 2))
 (segment (start 134.825 116.361) (end 134.981 116.205) (width 0.25) (layer "B.Cu") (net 2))
 (segment (start 147.175 120.904) (end 156.718 120.904) (width 0.25) (layer "B.Cu") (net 2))
 (segment (start 129.0001 116.361) (end 134.825 116.361) (width 0.25) (layer "B.Cu") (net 2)))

